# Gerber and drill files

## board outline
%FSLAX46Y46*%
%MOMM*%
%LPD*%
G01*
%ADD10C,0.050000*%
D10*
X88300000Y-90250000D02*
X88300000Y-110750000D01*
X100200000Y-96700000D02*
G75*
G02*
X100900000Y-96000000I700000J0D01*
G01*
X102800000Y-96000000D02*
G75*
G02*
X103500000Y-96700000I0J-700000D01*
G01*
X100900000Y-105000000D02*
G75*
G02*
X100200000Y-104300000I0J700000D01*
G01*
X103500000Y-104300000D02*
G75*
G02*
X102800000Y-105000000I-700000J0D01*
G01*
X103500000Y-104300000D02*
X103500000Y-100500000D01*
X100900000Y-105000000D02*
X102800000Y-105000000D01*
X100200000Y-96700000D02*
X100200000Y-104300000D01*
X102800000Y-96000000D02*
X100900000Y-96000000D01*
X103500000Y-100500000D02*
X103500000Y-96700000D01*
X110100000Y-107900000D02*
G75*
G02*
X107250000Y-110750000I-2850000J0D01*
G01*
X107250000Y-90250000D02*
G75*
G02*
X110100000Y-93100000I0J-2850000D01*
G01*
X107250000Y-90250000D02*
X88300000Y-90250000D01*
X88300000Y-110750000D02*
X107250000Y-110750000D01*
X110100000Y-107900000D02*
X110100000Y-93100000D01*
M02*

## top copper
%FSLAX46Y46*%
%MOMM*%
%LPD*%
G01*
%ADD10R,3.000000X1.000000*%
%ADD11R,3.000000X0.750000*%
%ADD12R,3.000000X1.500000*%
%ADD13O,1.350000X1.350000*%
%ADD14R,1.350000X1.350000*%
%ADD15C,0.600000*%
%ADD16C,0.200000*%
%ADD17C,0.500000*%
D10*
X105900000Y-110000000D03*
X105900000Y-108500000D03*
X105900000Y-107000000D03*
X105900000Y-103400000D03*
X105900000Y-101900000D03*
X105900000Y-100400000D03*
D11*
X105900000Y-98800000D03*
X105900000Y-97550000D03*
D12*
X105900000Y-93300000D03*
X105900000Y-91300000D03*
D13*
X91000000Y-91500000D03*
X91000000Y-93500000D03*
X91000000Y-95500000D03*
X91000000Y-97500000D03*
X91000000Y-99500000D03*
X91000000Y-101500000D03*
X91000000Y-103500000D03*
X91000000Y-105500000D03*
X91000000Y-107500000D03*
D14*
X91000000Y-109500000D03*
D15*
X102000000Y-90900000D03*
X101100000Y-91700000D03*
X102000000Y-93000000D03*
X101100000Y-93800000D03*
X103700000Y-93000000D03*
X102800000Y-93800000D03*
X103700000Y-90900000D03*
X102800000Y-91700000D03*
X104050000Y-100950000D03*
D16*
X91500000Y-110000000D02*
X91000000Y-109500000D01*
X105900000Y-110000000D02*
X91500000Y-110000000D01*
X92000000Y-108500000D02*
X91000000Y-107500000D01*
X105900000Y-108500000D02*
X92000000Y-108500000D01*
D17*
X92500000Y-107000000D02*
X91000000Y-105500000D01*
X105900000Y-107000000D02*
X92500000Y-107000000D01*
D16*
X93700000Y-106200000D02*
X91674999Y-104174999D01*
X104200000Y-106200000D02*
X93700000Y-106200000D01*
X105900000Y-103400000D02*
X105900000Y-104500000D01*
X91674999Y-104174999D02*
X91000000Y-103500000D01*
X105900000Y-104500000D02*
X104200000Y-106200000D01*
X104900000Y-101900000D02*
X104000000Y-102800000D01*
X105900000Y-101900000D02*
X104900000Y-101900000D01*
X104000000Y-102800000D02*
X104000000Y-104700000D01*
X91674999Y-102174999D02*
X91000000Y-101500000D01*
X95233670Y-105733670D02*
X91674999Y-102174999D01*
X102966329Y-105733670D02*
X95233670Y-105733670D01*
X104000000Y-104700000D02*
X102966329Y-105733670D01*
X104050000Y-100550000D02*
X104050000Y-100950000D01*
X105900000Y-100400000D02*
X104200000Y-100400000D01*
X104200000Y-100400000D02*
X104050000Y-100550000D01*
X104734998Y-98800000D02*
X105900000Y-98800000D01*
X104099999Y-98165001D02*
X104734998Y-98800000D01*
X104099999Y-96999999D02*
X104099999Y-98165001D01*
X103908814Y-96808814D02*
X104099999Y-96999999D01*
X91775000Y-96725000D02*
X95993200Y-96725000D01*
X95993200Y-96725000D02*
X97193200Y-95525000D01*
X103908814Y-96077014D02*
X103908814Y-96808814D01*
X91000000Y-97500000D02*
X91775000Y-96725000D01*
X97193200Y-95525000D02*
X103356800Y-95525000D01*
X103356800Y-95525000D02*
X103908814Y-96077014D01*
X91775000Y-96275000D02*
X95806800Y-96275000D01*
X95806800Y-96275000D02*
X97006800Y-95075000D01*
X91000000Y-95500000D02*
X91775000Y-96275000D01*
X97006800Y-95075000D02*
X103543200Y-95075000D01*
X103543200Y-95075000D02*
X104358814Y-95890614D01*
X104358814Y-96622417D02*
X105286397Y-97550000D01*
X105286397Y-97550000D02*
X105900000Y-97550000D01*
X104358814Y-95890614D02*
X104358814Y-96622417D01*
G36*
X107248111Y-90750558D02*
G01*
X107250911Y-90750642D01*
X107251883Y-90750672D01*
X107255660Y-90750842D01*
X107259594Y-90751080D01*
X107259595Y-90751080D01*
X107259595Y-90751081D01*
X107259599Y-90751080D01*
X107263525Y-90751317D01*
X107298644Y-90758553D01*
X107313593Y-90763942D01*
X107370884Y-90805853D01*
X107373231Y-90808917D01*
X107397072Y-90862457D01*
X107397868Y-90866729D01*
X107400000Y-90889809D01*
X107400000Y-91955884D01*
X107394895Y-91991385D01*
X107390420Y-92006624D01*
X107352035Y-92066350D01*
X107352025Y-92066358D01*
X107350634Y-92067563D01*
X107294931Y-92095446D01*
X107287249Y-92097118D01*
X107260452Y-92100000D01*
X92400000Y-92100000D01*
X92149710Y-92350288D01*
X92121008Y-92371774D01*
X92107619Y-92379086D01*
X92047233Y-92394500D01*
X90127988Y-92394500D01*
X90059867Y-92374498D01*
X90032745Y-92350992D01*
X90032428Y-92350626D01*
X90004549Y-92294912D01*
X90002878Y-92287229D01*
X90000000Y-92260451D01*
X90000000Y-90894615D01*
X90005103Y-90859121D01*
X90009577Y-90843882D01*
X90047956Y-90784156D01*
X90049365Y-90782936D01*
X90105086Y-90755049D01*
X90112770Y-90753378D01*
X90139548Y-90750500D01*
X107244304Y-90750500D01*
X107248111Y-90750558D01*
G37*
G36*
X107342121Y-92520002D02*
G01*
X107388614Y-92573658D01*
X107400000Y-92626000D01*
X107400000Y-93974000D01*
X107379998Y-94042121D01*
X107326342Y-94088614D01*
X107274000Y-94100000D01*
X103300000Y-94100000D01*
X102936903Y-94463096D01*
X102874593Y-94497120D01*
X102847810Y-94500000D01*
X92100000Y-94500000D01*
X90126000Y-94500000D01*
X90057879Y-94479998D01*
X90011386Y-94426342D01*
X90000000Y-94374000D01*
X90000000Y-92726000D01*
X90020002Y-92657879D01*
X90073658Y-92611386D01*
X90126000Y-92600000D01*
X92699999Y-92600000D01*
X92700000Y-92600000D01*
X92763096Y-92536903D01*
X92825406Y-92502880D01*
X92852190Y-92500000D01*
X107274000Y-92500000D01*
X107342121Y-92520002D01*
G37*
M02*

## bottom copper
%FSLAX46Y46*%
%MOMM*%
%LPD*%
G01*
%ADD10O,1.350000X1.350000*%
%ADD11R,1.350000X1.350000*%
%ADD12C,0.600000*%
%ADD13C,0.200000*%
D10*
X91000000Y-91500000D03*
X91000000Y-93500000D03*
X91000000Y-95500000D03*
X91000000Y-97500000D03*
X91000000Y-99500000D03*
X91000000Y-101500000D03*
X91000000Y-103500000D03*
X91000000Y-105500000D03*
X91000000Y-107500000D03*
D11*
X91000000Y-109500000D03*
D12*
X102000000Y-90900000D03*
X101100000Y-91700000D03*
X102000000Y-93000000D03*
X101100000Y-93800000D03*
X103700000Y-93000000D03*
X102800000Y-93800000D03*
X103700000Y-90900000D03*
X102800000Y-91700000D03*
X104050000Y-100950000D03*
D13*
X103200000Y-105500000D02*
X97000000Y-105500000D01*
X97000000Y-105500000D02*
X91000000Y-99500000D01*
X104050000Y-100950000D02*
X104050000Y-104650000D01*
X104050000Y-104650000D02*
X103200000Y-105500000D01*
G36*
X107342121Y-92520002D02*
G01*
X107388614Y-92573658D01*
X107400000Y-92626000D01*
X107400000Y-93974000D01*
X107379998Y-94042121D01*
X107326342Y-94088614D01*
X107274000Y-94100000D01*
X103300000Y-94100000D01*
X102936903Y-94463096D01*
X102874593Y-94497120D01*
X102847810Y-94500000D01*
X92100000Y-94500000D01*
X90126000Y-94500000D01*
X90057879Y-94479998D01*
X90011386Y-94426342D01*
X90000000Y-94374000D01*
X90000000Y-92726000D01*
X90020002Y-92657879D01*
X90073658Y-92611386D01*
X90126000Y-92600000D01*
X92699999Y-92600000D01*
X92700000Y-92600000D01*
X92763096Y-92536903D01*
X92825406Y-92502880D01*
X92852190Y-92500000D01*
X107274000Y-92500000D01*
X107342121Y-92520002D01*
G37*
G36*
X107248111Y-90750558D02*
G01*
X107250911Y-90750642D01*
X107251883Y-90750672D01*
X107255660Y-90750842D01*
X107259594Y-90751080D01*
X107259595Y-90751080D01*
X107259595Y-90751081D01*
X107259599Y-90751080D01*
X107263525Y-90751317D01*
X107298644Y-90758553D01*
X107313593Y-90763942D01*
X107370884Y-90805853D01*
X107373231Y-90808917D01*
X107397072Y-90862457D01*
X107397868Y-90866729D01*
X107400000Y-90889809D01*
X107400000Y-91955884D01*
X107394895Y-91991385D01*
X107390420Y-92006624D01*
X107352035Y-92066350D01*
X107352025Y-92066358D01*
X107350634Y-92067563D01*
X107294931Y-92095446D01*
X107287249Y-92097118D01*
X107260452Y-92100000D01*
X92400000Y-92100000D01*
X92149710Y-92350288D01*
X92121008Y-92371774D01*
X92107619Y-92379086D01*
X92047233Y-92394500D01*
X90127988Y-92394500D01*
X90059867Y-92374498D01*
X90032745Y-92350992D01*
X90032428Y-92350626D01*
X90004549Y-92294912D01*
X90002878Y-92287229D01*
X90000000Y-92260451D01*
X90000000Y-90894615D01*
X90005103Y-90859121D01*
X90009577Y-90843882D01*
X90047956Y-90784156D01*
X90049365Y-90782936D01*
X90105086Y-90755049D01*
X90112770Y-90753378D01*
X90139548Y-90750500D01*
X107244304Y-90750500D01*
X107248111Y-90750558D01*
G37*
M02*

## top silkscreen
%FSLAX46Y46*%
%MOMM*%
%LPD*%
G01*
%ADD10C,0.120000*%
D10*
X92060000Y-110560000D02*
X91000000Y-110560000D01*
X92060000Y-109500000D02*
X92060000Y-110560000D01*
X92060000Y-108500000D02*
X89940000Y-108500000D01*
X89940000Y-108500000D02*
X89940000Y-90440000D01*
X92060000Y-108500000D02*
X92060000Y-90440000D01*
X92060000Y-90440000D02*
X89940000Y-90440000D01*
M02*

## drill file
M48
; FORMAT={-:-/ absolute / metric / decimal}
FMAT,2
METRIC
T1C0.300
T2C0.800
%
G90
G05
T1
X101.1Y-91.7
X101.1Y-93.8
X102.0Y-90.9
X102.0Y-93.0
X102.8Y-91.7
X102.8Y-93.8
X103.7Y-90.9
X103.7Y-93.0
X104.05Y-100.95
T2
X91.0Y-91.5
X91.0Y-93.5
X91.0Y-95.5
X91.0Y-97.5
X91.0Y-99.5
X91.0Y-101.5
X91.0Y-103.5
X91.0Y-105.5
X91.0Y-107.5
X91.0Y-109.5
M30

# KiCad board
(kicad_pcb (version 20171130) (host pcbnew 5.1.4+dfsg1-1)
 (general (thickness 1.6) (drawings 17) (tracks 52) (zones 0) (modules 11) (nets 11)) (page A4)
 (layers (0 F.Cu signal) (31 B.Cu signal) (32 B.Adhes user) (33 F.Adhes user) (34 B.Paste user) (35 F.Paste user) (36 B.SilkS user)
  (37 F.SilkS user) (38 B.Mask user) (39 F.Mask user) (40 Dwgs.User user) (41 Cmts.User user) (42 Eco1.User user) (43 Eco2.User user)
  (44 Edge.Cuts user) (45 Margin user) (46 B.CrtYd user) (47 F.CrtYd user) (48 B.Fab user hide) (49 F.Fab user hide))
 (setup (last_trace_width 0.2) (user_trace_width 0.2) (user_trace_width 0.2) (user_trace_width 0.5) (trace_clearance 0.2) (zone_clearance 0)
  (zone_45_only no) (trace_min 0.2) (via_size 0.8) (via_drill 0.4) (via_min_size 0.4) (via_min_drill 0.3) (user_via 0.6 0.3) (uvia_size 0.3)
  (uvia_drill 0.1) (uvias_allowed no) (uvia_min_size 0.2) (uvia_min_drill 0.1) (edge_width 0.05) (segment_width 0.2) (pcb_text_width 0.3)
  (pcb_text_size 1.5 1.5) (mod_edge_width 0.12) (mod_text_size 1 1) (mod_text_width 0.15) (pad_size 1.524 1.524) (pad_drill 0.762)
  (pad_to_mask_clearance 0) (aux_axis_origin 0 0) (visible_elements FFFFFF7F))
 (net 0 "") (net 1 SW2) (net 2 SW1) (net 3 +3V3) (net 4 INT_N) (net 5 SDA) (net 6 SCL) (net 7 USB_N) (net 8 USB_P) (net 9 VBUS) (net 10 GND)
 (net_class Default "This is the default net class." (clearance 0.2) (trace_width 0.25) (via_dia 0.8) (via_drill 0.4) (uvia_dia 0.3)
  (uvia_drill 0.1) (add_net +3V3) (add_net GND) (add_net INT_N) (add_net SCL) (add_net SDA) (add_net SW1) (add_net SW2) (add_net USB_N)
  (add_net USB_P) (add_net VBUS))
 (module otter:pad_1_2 (layer F.Cu) (at 105.9 110 90)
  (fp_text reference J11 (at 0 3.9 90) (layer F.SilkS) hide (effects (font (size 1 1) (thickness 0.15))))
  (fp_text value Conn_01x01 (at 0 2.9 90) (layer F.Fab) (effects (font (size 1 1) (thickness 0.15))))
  (pad 1 smd rect (at 0 0 90) (size 1 3) (layers F.Cu F.Paste F.Mask) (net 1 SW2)))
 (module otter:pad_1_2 (layer F.Cu) (at 105.9 108.5 90)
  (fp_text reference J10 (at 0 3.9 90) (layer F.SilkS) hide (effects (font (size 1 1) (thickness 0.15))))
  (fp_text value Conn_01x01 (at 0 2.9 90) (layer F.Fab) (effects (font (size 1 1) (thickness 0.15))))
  (pad 1 smd rect (at 0 0 90) (size 1 3) (layers F.Cu F.Paste F.Mask) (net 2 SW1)))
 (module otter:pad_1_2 (layer F.Cu) (at 105.9 107 90)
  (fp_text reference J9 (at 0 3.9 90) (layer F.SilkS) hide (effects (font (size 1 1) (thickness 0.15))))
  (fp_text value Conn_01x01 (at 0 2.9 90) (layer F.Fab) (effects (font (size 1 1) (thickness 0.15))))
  (pad 1 smd rect (at 0 0 90) (size 1 3) (layers F.Cu F.Paste F.Mask) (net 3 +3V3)))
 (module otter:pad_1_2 (layer F.Cu) (at 105.9 103.4 90)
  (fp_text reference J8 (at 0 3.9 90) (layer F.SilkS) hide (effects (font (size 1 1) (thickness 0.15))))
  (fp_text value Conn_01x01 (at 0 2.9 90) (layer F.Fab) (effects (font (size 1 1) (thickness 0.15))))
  (pad 1 smd rect (at 0 0 90) (size 1 3) (layers F.Cu F.Paste F.Mask) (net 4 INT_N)))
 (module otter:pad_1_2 (layer F.Cu) (at 105.9 101.9 90)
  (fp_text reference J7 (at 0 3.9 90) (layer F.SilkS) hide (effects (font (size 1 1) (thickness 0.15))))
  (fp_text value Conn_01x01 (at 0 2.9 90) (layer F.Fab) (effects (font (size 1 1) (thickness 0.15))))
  (pad 1 smd rect (at 0 0 90) (size 1 3) (layers F.Cu F.Paste F.Mask) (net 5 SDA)))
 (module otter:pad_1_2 (layer F.Cu) (at 105.9 100.4 90)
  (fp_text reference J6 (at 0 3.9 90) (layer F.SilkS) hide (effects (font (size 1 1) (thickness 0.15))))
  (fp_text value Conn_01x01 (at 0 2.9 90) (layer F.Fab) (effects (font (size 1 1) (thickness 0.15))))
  (pad 1 smd rect (at 0 0 90) (size 1 3) (layers F.Cu F.Paste F.Mask) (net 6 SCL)))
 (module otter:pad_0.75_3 (layer F.Cu) (at 105.9 98.8 90)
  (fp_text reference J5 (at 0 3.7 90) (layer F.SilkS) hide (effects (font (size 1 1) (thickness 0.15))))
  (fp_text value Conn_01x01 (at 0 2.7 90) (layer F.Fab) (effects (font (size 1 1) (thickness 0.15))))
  (pad 1 smd rect (at 0 0 90) (size 0.75 3) (layers F.Cu F.Paste F.Mask) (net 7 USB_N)))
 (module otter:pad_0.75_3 (layer F.Cu) (at 105.9 97.55 90)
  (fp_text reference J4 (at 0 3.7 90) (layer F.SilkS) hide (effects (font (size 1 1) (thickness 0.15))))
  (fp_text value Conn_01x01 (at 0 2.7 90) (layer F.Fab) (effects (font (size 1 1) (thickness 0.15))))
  (pad 1 smd rect (at 0 0 90) (size 0.75 3) (layers F.Cu F.Paste F.Mask) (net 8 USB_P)))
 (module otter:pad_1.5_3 (layer F.Cu) (at 105.9 93.3 90)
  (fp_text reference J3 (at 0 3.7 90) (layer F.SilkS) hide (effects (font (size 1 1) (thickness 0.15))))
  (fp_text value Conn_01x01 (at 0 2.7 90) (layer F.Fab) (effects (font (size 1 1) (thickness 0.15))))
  (pad 1 smd rect (at 0 0 90) (size 1.5 3) (layers F.Cu F.Paste F.Mask) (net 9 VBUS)))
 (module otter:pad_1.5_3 (layer F.Cu) (at 105.9 91.3 90)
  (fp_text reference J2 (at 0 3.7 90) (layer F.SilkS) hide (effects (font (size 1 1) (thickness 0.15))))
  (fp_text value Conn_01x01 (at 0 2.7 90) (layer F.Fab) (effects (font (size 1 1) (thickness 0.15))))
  (pad 1 smd rect (at 0 0 90) (size 1.5 3) (layers F.Cu F.Paste F.Mask) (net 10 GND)))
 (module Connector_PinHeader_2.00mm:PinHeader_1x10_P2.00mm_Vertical (layer F.Cu) (at 91 100.5 180)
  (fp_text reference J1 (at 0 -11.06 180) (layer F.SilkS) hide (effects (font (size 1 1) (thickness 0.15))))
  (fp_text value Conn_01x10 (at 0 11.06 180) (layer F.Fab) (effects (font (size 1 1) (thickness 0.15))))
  (fp_line (start -1.06 -10.06) (end 0 -10.06) (layer F.SilkS) (width 0.12))
  (fp_line (start -1.06 -9) (end -1.06 -10.06) (layer F.SilkS) (width 0.12))
  (fp_line (start -1.06 -8) (end 1.06 -8) (layer F.SilkS) (width 0.12))
  (fp_line (start 1.06 -8) (end 1.06 10.06) (layer F.SilkS) (width 0.12))
  (fp_line (start -1.06 -8) (end -1.06 10.06) (layer F.SilkS) (width 0.12))
  (fp_line (start -1.06 10.06) (end 1.06 10.06) (layer F.SilkS) (width 0.12))
  (pad 10 thru_hole oval (at 0 9 180) (size 1.35 1.35) (drill 0.8) (layers *.Cu *.Mask) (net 10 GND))
  (pad 9 thru_hole oval (at 0 7 180) (size 1.35 1.35) (drill 0.8) (layers *.Cu *.Mask) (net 9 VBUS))
  (pad 8 thru_hole oval (at 0 5 180) (size 1.35 1.35) (drill 0.8) (layers *.Cu *.Mask) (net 8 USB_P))
  (pad 7 thru_hole oval (at 0 3 180) (size 1.35 1.35) (drill 0.8) (layers *.Cu *.Mask) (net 7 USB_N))
  (pad 6 thru_hole oval (at 0 1 180) (size 1.35 1.35) (drill 0.8) (layers *.Cu *.Mask) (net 6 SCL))
  (pad 5 thru_hole oval (at 0 -1 180) (size 1.35 1.35) (drill 0.8) (layers *.Cu *.Mask) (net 5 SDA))
  (pad 4 thru_hole oval (at 0 -3 180) (size 1.35 1.35) (drill 0.8) (layers *.Cu *.Mask) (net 4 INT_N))
  (pad 3 thru_hole oval (at 0 -5 180) (size 1.35 1.35) (drill 0.8) (layers *.Cu *.Mask) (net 3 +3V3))
  (pad 2 thru_hole oval (at 0 -7 180) (size 1.35 1.35) (drill 0.8) (layers *.Cu *.Mask) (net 2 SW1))
  (pad 1 thru_hole rect (at 0 -9 180) (size 1.35 1.35) (drill 0.8) (layers *.Cu *.Mask) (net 1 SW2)))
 (gr_line (start 88.3 90.25) (end 88.3 110.75) (layer Edge.Cuts) (width 0.05))
 (gr_arc (start 100.9 96.7) (end 100.9 96) (angle -90) (layer Edge.Cuts) (width 0.05))
 (gr_arc (start 102.8 96.7) (end 103.5 96.7) (angle -90) (layer Edge.Cuts) (width 0.05))
 (gr_arc (start 100.9 104.3) (end 100.2 104.3) (angle -90) (layer Edge.Cuts) (width 0.05))
 (gr_arc (start 102.8 104.3) (end 102.8 105) (angle -90) (layer Edge.Cuts) (width 0.05))
 (gr_line (start 103.5 104.3) (end 103.5 100.5) (layer Edge.Cuts) (width 0.05))
 (gr_line (start 100.9 105) (end 102.8 105) (layer Edge.Cuts) (width 0.05))
 (gr_line (start 100.2 96.7) (end 100.2 104.3) (layer Edge.Cuts) (width 0.05))
 (gr_line (start 102.8 96) (end 100.9 96) (layer Edge.Cuts) (width 0.05))
 (gr_line (start 103.5 100.5) (end 103.5 96.7) (layer Edge.Cuts) (width 0.05))
 (gr_arc (start 107.25 107.9) (end 107.25 110.75) (angle -90) (layer Edge.Cuts) (width 0.05))
 (gr_arc (start 107.25 93.1) (end 110.1 93.1) (angle -90) (layer Edge.Cuts) (width 0.05))
 (gr_line (start 107.25 90.25) (end 88.3 90.25) (layer Edge.Cuts) (width 0.05))
 (gr_line (start 88.3 110.75) (end 107.25 110.75) (layer Edge.Cuts) (width 0.05))
 (gr_line (start 110.1 107.9) (end 110.1 93.1) (layer Edge.Cuts) (width 0.05))
 (via (at 102 90.9) (size 0.6) (drill 0.3) (layers F.Cu B.Cu) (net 10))
 (via (at 101.1 91.7) (size 0.6) (drill 0.3) (layers F.Cu B.Cu) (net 10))
 (via (at 102 93) (size 0.6) (drill 0.3) (layers F.Cu B.Cu) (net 9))
 (via (at 101.1 93.8) (size 0.6) (drill 0.3) (layers F.Cu B.Cu) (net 9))
 (via (at 103.7 93) (size 0.6) (drill 0.3) (layers F.Cu B.Cu) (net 9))
 (via (at 102.8 93.8) (size 0.6) (drill 0.3) (layers F.Cu B.Cu) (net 9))
 (via (at 103.7 90.9) (size 0.6) (drill 0.3) (layers F.Cu B.Cu) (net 10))
 (via (at 102.8 91.7) (size 0.6) (drill 0.3) (layers F.Cu B.Cu) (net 10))
 (segment (start 91.5 110) (end 91 109.5) (width 0.2) (layer F.Cu) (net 1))
 (segment (start 105.9 110) (end 91.5 110) (width 0.2) (layer F.Cu) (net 1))
 (segment (start 92 108.5) (end 91 107.5) (width 0.2) (layer F.Cu) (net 2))
 (segment (start 105.9 108.5) (end 92 108.5) (width 0.2) (layer F.Cu) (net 2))
 (segment (start 92.5 107) (end 91 105.5) (width 0.5) (layer F.Cu) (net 3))
 (segment (start 105.9 107) (end 92.5 107) (width 0.5) (layer F.Cu) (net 3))
 (segment (start 93.7 106.2) (end 91.674999 104.174999) (width 0.2) (layer F.Cu) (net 4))
 (segment (start 104.2 106.2) (end 93.7 106.2) (width 0.2) (layer F.Cu) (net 4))
 (segment (start 105.9 103.4) (end 105.9 104.5) (width 0.2) (layer F.Cu) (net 4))
 (segment (start 91.674999 104.174999) (end 91 103.5) (width 0.2) (layer F.Cu) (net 4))
 (segment (start 105.9 104.5) (end 104.2 106.2) (width 0.2) (layer F.Cu) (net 4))
 (segment (start 104.9 101.9) (end 104 102.8) (width 0.2) (layer F.Cu) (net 5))
 (segment (start 105.9 101.9) (end 104.9 101.9) (width 0.2) (layer F.Cu) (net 5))
 (segment (start 104 102.8) (end 104 104.7) (width 0.2) (layer F.Cu) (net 5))
 (segment (start 91.674999 102.174999) (end 91 101.5) (width 0.2) (layer F.Cu) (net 5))
 (segment (start 95.23367 105.73367) (end 91.674999 102.174999) (width 0.2) (layer F.Cu) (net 5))
 (segment (start 102.966329 105.73367) (end 95.23367 105.73367) (width 0.2) (layer F.Cu) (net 5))
 (segment (start 104 104.7) (end 102.966329 105.73367) (width 0.2) (layer F.Cu) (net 5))
 (via (at 104.05 100.95) (size 0.6) (drill 0.3) (layers F.Cu B.Cu) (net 6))
 (segment (start 104.05 100.55) (end 104.05 100.95) (width 0.2) (layer F.Cu) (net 6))
 (segment (start 105.9 100.4) (end 104.2 100.4) (width 0.2) (layer F.Cu) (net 6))
 (segment (start 104.2 100.4) (end 104.05 100.55) (width 0.2) (layer F.Cu) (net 6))
 (segment (start 103.2 105.5) (end 97 105.5) (width 0.2) (layer B.Cu) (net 6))
 (segment (start 97 105.5) (end 91 99.5) (width 0.2) (layer B.Cu) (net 6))
 (segment (start 104.05 100.95) (end 104.05 104.65) (width 0.2) (layer B.Cu) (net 6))
 (segment (start 104.05 104.65) (end 103.2 105.5) (width 0.2) (layer B.Cu) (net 6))
 (segment (start 104.734998 98.8) (end 105.9 98.8) (width 0.2) (layer F.Cu) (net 7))
 (segment (start 104.099999 98.165001) (end 104.734998 98.8) (width 0.2) (layer F.Cu) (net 7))
 (segment (start 104.099999 96.999999) (end 104.099999 98.165001) (width 0.2) (layer F.Cu) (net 7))
 (segment (start 103.908814 96.808814) (end 104.099999 96.999999) (width 0.2) (layer F.Cu) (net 7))
 (segment (start 91.775 96.725) (end 95.9932 96.725) (width 0.2) (layer F.Cu) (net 7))
 (segment (start 95.9932 96.725) (end 97.1932 95.525) (width 0.2) (layer F.Cu) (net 7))
 (segment (start 103.908814 96.077014) (end 103.908814 96.808814) (width 0.2) (layer F.Cu) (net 7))
 (segment (start 91 97.5) (end 91.775 96.725) (width 0.2) (layer F.Cu) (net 7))
 (segment (start 97.1932 95.525) (end 103.3568 95.525) (width 0.2) (layer F.Cu) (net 7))
 (segment (start 103.3568 95.525) (end 103.908814 96.077014) (width 0.2) (layer F.Cu) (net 7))
 (segment (start 91.775 96.275) (end 95.8068 96.275) (width 0.2) (layer F.Cu) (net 8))
 (segment (start 95.8068 96.275) (end 97.0068 95.075) (width 0.2) (layer F.Cu) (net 8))
 (segment (start 91 95.5) (end 91.775 96.275) (width 0.2) (layer F.Cu) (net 8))
 (segment (start 97.0068 95.075) (end 103.5432 95.075) (width 0.2) (layer F.Cu) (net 8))
 (segment (start 103.5432 95.075) (end 104.358814 95.890614) (width 0.2) (layer F.Cu) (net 8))
 (segment (start 104.358814 96.622417) (end 105.286397 97.55) (width 0.2) (layer F.Cu) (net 8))
 (segment (start 105.286397 97.55) (end 105.9 97.55) (width 0.2) (layer F.Cu) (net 8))
 (segment (start 104.358814 95.890614) (end 104.358814 96.622417) (width 0.2) (layer F.Cu) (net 8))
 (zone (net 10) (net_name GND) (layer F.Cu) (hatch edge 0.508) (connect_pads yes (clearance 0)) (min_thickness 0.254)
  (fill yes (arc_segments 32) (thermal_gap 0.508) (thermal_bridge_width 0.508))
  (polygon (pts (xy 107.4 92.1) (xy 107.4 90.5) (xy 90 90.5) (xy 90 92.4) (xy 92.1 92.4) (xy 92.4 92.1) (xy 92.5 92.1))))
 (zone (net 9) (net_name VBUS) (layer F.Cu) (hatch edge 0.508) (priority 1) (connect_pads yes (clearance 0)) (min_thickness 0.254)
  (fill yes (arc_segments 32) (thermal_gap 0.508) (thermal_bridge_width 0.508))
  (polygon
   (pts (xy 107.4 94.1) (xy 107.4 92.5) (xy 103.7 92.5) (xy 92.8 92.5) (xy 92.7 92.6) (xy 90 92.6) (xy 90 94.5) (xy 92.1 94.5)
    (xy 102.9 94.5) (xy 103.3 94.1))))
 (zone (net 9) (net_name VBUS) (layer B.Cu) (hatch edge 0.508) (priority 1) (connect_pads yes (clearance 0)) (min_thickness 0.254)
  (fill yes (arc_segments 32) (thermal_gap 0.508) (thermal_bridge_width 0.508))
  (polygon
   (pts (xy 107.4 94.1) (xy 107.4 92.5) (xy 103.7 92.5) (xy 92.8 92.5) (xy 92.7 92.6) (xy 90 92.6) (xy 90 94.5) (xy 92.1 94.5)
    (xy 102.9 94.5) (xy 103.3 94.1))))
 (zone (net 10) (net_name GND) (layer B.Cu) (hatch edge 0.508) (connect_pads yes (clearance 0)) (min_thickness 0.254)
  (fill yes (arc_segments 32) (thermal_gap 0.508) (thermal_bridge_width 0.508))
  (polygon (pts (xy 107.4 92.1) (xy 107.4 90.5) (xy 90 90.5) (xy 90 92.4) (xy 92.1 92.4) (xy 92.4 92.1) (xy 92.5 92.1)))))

